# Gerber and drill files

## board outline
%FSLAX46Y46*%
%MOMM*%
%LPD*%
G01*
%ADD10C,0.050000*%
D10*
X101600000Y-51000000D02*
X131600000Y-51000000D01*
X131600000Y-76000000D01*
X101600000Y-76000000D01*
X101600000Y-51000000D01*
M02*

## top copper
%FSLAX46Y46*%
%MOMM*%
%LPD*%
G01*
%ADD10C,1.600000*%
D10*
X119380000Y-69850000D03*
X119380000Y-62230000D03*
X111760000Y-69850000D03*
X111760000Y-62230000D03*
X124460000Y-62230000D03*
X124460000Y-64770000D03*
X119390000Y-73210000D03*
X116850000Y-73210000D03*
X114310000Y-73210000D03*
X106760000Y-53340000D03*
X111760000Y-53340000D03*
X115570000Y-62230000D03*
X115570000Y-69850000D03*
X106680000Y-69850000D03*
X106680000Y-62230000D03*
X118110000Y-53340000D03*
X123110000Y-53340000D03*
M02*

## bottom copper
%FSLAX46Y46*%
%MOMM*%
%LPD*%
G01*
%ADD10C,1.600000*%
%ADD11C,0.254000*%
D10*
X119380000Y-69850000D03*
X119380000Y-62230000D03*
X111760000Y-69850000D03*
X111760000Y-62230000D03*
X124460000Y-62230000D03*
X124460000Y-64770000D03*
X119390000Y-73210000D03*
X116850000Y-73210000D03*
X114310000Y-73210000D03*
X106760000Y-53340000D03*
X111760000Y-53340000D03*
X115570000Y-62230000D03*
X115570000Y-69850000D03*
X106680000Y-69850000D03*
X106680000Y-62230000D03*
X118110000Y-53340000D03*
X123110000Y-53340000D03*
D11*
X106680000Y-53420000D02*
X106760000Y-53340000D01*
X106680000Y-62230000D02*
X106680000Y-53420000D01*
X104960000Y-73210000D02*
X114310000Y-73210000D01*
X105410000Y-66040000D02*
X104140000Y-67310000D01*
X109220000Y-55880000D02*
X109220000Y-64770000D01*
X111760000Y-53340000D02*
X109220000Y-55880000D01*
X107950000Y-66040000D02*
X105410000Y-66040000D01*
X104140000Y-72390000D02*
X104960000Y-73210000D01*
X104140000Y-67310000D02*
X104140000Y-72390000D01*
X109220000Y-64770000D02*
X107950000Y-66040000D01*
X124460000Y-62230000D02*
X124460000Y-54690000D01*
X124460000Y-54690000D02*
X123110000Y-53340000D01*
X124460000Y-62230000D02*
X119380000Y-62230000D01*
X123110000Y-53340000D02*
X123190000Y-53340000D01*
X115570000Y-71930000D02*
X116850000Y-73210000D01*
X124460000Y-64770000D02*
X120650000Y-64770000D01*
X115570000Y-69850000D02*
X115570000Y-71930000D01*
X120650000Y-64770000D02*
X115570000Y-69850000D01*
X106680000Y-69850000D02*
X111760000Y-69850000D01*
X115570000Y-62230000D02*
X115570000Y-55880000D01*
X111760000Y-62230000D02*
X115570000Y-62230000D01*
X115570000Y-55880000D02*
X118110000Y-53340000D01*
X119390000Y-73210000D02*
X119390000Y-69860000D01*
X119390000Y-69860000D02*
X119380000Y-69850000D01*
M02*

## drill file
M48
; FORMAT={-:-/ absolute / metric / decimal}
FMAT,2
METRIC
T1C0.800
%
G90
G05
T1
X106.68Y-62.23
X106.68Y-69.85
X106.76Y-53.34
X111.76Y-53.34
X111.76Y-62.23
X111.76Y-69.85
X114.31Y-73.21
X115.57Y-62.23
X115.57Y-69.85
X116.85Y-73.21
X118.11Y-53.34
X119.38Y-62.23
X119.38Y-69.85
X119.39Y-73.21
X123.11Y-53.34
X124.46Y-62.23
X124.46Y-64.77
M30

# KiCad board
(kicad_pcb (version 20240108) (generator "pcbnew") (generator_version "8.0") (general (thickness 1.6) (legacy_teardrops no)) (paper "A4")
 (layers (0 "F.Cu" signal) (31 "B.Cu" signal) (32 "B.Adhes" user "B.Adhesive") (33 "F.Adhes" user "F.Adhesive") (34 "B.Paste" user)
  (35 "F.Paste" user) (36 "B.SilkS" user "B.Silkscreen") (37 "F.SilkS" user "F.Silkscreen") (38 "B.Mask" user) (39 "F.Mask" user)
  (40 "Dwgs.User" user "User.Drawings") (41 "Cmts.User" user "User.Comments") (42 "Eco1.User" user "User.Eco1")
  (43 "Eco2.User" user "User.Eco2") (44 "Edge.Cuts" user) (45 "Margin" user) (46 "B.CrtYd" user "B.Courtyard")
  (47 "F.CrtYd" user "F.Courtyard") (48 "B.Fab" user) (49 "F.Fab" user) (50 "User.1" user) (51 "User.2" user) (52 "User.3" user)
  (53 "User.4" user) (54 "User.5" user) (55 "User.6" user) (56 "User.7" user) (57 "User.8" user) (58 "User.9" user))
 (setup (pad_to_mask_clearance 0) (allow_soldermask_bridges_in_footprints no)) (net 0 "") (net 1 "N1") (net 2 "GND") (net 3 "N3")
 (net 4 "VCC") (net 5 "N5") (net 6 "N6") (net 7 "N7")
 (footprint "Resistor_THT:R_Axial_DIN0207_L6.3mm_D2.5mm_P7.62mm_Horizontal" (layer "F.Cu") (at 119.38 69.85 90)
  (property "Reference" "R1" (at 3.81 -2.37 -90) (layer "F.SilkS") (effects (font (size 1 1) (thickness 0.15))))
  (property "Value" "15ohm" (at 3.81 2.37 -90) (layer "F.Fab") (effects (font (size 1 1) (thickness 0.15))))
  (pad "1" thru_hole circle (at 0 0 90) (size 1.6 1.6) (drill 0.8) (layers "*.Cu" "*.Mask") (remove_unused_layers no) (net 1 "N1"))
  (pad "2" thru_hole circle (at 7.62 0 90) (size 1.6 1.6) (drill 0.8) (layers "*.Cu" "*.Mask") (remove_unused_layers no) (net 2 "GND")))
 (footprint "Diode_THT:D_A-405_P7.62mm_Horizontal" (layer "F.Cu") (at 111.76 69.85 90)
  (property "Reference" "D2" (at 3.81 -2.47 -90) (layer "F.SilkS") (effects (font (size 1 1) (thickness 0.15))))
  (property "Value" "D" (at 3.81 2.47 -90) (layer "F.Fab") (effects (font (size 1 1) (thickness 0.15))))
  (pad "1" thru_hole circle (at 0 0 90) (size 1.6 1.6) (drill 0.8) (layers "*.Cu" "*.Mask") (remove_unused_layers no) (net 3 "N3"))
  (pad "2" thru_hole circle (at 7.62 0 90) (size 1.6 1.6) (drill 0.8) (layers "*.Cu" "*.Mask") (remove_unused_layers no) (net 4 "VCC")))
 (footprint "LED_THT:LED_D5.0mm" (layer "F.Cu") (at 124.46 62.23 -90)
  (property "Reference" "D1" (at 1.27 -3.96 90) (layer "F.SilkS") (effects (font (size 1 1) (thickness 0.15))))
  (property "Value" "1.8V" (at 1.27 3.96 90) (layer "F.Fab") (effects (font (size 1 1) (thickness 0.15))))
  (pad "1" thru_hole circle (at 0 0 270) (size 1.6 1.6) (drill 0.8) (layers "*.Cu" "*.Mask") (remove_unused_layers no) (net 2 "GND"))
  (pad "2" thru_hole circle (at 2.54 0 270) (size 1.6 1.6) (drill 0.8) (layers "*.Cu" "*.Mask") (remove_unused_layers no) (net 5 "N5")))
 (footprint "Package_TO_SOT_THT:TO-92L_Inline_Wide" (layer "F.Cu") (at 119.39 73.21 180)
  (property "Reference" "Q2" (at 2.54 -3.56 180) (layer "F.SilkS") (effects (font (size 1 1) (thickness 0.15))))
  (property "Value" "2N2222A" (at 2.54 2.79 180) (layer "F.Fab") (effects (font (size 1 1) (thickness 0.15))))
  (pad "1" thru_hole circle (at 0 0 180) (size 1.6 1.6) (drill 0.8) (layers "*.Cu" "*.Mask") (remove_unused_layers no) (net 1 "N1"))
  (pad "2" thru_hole circle (at 2.54 0 180) (size 1.6 1.6) (drill 0.8) (layers "*.Cu" "*.Mask") (remove_unused_layers no) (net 5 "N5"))
  (pad "3" thru_hole circle (at 5.08 0 180) (size 1.6 1.6) (drill 0.8) (layers "*.Cu" "*.Mask") (remove_unused_layers no) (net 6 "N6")))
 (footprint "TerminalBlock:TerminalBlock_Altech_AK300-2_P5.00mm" (layer "F.Cu") (at 106.76 53.34)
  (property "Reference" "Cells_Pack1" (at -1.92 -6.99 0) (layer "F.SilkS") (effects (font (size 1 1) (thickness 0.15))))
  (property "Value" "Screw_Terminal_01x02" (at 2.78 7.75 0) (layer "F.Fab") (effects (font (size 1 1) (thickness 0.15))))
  (pad "1" thru_hole circle (at 0 0) (size 1.6 1.6) (drill 0.8) (layers "*.Cu" "*.Mask") (remove_unused_layers no) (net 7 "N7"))
  (pad "2" thru_hole circle (at 5 0) (size 1.6 1.6) (drill 0.8) (layers "*.Cu" "*.Mask") (remove_unused_layers no) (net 6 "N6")))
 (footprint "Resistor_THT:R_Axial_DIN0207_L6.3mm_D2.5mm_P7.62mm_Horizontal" (layer "F.Cu") (at 115.57 62.23 -90)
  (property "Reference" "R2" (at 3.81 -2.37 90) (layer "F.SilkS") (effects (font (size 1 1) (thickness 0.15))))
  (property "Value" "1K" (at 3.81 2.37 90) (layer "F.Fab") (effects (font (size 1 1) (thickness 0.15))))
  (pad "1" thru_hole circle (at 0 0 270) (size 1.6 1.6) (drill 0.8) (layers "*.Cu" "*.Mask") (remove_unused_layers no) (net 4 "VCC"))
  (pad "2" thru_hole circle (at 7.62 0 270) (size 1.6 1.6) (drill 0.8) (layers "*.Cu" "*.Mask") (remove_unused_layers no) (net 5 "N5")))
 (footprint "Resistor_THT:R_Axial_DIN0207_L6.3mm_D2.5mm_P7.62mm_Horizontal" (layer "F.Cu") (at 106.68 69.85 90)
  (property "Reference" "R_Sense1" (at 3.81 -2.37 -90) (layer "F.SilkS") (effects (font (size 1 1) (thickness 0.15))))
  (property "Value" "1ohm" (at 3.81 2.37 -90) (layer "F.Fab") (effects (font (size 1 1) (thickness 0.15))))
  (pad "1" thru_hole circle (at 0 0 90) (size 1.6 1.6) (drill 0.8) (layers "*.Cu" "*.Mask") (remove_unused_layers no) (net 3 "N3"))
  (pad "2" thru_hole circle (at 7.62 0 90) (size 1.6 1.6) (drill 0.8) (layers "*.Cu" "*.Mask") (remove_unused_layers no) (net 7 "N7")))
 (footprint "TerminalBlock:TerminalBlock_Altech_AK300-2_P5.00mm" (layer "F.Cu") (at 118.11 53.34)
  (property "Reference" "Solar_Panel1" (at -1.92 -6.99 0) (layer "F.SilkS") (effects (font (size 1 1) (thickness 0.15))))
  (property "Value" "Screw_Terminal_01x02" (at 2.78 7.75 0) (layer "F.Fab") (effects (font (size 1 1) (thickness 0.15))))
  (pad "1" thru_hole circle (at 0 0) (size 1.6 1.6) (drill 0.8) (layers "*.Cu" "*.Mask") (remove_unused_layers no) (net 4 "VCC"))
  (pad "2" thru_hole circle (at 5 0) (size 1.6 1.6) (drill 0.8) (layers "*.Cu" "*.Mask") (remove_unused_layers no) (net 2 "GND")))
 (gr_rect (start 101.6 51) (end 131.6 76) (stroke (width 0.05) (type default)) (fill none) (layer "Edge.Cuts"))
 (segment (start 106.68 53.42) (end 106.76 53.34) (width 0.254) (layer "B.Cu") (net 7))
 (segment (start 106.68 62.23) (end 106.68 53.42) (width 0.254) (layer "B.Cu") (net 7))
 (segment (start 104.96 73.21) (end 114.31 73.21) (width 0.254) (layer "B.Cu") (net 6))
 (segment (start 105.41 66.04) (end 104.14 67.31) (width 0.254) (layer "B.Cu") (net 6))
 (segment (start 109.22 55.88) (end 109.22 64.77) (width 0.254) (layer "B.Cu") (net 6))
 (segment (start 111.76 53.34) (end 109.22 55.88) (width 0.254) (layer "B.Cu") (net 6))
 (segment (start 107.95 66.04) (end 105.41 66.04) (width 0.254) (layer "B.Cu") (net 6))
 (segment (start 104.14 72.39) (end 104.96 73.21) (width 0.254) (layer "B.Cu") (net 6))
 (segment (start 104.14 67.31) (end 104.14 72.39) (width 0.254) (layer "B.Cu") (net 6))
 (segment (start 109.22 64.77) (end 107.95 66.04) (width 0.254) (layer "B.Cu") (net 6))
 (segment (start 124.46 62.23) (end 124.46 54.69) (width 0.254) (layer "B.Cu") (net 2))
 (segment (start 124.46 54.69) (end 123.11 53.34) (width 0.254) (layer "B.Cu") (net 2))
 (segment (start 124.46 62.23) (end 119.38 62.23) (width 0.254) (layer "B.Cu") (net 2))
 (segment (start 123.11 53.34) (end 123.19 53.34) (width 0.254) (layer "B.Cu") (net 2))
 (segment (start 115.57 71.93) (end 116.85 73.21) (width 0.254) (layer "B.Cu") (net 5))
 (segment (start 124.46 64.77) (end 120.65 64.77) (width 0.254) (layer "B.Cu") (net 5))
 (segment (start 115.57 69.85) (end 115.57 71.93) (width 0.254) (layer "B.Cu") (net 5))
 (segment (start 120.65 64.77) (end 115.57 69.85) (width 0.254) (layer "B.Cu") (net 5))
 (segment (start 106.68 69.85) (end 111.76 69.85) (width 0.254) (layer "B.Cu") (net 3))
 (segment (start 115.57 62.23) (end 115.57 55.88) (width 0.254) (layer "B.Cu") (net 4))
 (segment (start 111.76 62.23) (end 115.57 62.23) (width 0.254) (layer "B.Cu") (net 4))
 (segment (start 115.57 55.88) (end 118.11 53.34) (width 0.254) (layer "B.Cu") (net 4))
 (segment (start 119.39 73.21) (end 119.39 69.86) (width 0.254) (layer "B.Cu") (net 1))
 (segment (start 119.39 69.86) (end 119.38 69.85) (width 0.254) (layer "B.Cu") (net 1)))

